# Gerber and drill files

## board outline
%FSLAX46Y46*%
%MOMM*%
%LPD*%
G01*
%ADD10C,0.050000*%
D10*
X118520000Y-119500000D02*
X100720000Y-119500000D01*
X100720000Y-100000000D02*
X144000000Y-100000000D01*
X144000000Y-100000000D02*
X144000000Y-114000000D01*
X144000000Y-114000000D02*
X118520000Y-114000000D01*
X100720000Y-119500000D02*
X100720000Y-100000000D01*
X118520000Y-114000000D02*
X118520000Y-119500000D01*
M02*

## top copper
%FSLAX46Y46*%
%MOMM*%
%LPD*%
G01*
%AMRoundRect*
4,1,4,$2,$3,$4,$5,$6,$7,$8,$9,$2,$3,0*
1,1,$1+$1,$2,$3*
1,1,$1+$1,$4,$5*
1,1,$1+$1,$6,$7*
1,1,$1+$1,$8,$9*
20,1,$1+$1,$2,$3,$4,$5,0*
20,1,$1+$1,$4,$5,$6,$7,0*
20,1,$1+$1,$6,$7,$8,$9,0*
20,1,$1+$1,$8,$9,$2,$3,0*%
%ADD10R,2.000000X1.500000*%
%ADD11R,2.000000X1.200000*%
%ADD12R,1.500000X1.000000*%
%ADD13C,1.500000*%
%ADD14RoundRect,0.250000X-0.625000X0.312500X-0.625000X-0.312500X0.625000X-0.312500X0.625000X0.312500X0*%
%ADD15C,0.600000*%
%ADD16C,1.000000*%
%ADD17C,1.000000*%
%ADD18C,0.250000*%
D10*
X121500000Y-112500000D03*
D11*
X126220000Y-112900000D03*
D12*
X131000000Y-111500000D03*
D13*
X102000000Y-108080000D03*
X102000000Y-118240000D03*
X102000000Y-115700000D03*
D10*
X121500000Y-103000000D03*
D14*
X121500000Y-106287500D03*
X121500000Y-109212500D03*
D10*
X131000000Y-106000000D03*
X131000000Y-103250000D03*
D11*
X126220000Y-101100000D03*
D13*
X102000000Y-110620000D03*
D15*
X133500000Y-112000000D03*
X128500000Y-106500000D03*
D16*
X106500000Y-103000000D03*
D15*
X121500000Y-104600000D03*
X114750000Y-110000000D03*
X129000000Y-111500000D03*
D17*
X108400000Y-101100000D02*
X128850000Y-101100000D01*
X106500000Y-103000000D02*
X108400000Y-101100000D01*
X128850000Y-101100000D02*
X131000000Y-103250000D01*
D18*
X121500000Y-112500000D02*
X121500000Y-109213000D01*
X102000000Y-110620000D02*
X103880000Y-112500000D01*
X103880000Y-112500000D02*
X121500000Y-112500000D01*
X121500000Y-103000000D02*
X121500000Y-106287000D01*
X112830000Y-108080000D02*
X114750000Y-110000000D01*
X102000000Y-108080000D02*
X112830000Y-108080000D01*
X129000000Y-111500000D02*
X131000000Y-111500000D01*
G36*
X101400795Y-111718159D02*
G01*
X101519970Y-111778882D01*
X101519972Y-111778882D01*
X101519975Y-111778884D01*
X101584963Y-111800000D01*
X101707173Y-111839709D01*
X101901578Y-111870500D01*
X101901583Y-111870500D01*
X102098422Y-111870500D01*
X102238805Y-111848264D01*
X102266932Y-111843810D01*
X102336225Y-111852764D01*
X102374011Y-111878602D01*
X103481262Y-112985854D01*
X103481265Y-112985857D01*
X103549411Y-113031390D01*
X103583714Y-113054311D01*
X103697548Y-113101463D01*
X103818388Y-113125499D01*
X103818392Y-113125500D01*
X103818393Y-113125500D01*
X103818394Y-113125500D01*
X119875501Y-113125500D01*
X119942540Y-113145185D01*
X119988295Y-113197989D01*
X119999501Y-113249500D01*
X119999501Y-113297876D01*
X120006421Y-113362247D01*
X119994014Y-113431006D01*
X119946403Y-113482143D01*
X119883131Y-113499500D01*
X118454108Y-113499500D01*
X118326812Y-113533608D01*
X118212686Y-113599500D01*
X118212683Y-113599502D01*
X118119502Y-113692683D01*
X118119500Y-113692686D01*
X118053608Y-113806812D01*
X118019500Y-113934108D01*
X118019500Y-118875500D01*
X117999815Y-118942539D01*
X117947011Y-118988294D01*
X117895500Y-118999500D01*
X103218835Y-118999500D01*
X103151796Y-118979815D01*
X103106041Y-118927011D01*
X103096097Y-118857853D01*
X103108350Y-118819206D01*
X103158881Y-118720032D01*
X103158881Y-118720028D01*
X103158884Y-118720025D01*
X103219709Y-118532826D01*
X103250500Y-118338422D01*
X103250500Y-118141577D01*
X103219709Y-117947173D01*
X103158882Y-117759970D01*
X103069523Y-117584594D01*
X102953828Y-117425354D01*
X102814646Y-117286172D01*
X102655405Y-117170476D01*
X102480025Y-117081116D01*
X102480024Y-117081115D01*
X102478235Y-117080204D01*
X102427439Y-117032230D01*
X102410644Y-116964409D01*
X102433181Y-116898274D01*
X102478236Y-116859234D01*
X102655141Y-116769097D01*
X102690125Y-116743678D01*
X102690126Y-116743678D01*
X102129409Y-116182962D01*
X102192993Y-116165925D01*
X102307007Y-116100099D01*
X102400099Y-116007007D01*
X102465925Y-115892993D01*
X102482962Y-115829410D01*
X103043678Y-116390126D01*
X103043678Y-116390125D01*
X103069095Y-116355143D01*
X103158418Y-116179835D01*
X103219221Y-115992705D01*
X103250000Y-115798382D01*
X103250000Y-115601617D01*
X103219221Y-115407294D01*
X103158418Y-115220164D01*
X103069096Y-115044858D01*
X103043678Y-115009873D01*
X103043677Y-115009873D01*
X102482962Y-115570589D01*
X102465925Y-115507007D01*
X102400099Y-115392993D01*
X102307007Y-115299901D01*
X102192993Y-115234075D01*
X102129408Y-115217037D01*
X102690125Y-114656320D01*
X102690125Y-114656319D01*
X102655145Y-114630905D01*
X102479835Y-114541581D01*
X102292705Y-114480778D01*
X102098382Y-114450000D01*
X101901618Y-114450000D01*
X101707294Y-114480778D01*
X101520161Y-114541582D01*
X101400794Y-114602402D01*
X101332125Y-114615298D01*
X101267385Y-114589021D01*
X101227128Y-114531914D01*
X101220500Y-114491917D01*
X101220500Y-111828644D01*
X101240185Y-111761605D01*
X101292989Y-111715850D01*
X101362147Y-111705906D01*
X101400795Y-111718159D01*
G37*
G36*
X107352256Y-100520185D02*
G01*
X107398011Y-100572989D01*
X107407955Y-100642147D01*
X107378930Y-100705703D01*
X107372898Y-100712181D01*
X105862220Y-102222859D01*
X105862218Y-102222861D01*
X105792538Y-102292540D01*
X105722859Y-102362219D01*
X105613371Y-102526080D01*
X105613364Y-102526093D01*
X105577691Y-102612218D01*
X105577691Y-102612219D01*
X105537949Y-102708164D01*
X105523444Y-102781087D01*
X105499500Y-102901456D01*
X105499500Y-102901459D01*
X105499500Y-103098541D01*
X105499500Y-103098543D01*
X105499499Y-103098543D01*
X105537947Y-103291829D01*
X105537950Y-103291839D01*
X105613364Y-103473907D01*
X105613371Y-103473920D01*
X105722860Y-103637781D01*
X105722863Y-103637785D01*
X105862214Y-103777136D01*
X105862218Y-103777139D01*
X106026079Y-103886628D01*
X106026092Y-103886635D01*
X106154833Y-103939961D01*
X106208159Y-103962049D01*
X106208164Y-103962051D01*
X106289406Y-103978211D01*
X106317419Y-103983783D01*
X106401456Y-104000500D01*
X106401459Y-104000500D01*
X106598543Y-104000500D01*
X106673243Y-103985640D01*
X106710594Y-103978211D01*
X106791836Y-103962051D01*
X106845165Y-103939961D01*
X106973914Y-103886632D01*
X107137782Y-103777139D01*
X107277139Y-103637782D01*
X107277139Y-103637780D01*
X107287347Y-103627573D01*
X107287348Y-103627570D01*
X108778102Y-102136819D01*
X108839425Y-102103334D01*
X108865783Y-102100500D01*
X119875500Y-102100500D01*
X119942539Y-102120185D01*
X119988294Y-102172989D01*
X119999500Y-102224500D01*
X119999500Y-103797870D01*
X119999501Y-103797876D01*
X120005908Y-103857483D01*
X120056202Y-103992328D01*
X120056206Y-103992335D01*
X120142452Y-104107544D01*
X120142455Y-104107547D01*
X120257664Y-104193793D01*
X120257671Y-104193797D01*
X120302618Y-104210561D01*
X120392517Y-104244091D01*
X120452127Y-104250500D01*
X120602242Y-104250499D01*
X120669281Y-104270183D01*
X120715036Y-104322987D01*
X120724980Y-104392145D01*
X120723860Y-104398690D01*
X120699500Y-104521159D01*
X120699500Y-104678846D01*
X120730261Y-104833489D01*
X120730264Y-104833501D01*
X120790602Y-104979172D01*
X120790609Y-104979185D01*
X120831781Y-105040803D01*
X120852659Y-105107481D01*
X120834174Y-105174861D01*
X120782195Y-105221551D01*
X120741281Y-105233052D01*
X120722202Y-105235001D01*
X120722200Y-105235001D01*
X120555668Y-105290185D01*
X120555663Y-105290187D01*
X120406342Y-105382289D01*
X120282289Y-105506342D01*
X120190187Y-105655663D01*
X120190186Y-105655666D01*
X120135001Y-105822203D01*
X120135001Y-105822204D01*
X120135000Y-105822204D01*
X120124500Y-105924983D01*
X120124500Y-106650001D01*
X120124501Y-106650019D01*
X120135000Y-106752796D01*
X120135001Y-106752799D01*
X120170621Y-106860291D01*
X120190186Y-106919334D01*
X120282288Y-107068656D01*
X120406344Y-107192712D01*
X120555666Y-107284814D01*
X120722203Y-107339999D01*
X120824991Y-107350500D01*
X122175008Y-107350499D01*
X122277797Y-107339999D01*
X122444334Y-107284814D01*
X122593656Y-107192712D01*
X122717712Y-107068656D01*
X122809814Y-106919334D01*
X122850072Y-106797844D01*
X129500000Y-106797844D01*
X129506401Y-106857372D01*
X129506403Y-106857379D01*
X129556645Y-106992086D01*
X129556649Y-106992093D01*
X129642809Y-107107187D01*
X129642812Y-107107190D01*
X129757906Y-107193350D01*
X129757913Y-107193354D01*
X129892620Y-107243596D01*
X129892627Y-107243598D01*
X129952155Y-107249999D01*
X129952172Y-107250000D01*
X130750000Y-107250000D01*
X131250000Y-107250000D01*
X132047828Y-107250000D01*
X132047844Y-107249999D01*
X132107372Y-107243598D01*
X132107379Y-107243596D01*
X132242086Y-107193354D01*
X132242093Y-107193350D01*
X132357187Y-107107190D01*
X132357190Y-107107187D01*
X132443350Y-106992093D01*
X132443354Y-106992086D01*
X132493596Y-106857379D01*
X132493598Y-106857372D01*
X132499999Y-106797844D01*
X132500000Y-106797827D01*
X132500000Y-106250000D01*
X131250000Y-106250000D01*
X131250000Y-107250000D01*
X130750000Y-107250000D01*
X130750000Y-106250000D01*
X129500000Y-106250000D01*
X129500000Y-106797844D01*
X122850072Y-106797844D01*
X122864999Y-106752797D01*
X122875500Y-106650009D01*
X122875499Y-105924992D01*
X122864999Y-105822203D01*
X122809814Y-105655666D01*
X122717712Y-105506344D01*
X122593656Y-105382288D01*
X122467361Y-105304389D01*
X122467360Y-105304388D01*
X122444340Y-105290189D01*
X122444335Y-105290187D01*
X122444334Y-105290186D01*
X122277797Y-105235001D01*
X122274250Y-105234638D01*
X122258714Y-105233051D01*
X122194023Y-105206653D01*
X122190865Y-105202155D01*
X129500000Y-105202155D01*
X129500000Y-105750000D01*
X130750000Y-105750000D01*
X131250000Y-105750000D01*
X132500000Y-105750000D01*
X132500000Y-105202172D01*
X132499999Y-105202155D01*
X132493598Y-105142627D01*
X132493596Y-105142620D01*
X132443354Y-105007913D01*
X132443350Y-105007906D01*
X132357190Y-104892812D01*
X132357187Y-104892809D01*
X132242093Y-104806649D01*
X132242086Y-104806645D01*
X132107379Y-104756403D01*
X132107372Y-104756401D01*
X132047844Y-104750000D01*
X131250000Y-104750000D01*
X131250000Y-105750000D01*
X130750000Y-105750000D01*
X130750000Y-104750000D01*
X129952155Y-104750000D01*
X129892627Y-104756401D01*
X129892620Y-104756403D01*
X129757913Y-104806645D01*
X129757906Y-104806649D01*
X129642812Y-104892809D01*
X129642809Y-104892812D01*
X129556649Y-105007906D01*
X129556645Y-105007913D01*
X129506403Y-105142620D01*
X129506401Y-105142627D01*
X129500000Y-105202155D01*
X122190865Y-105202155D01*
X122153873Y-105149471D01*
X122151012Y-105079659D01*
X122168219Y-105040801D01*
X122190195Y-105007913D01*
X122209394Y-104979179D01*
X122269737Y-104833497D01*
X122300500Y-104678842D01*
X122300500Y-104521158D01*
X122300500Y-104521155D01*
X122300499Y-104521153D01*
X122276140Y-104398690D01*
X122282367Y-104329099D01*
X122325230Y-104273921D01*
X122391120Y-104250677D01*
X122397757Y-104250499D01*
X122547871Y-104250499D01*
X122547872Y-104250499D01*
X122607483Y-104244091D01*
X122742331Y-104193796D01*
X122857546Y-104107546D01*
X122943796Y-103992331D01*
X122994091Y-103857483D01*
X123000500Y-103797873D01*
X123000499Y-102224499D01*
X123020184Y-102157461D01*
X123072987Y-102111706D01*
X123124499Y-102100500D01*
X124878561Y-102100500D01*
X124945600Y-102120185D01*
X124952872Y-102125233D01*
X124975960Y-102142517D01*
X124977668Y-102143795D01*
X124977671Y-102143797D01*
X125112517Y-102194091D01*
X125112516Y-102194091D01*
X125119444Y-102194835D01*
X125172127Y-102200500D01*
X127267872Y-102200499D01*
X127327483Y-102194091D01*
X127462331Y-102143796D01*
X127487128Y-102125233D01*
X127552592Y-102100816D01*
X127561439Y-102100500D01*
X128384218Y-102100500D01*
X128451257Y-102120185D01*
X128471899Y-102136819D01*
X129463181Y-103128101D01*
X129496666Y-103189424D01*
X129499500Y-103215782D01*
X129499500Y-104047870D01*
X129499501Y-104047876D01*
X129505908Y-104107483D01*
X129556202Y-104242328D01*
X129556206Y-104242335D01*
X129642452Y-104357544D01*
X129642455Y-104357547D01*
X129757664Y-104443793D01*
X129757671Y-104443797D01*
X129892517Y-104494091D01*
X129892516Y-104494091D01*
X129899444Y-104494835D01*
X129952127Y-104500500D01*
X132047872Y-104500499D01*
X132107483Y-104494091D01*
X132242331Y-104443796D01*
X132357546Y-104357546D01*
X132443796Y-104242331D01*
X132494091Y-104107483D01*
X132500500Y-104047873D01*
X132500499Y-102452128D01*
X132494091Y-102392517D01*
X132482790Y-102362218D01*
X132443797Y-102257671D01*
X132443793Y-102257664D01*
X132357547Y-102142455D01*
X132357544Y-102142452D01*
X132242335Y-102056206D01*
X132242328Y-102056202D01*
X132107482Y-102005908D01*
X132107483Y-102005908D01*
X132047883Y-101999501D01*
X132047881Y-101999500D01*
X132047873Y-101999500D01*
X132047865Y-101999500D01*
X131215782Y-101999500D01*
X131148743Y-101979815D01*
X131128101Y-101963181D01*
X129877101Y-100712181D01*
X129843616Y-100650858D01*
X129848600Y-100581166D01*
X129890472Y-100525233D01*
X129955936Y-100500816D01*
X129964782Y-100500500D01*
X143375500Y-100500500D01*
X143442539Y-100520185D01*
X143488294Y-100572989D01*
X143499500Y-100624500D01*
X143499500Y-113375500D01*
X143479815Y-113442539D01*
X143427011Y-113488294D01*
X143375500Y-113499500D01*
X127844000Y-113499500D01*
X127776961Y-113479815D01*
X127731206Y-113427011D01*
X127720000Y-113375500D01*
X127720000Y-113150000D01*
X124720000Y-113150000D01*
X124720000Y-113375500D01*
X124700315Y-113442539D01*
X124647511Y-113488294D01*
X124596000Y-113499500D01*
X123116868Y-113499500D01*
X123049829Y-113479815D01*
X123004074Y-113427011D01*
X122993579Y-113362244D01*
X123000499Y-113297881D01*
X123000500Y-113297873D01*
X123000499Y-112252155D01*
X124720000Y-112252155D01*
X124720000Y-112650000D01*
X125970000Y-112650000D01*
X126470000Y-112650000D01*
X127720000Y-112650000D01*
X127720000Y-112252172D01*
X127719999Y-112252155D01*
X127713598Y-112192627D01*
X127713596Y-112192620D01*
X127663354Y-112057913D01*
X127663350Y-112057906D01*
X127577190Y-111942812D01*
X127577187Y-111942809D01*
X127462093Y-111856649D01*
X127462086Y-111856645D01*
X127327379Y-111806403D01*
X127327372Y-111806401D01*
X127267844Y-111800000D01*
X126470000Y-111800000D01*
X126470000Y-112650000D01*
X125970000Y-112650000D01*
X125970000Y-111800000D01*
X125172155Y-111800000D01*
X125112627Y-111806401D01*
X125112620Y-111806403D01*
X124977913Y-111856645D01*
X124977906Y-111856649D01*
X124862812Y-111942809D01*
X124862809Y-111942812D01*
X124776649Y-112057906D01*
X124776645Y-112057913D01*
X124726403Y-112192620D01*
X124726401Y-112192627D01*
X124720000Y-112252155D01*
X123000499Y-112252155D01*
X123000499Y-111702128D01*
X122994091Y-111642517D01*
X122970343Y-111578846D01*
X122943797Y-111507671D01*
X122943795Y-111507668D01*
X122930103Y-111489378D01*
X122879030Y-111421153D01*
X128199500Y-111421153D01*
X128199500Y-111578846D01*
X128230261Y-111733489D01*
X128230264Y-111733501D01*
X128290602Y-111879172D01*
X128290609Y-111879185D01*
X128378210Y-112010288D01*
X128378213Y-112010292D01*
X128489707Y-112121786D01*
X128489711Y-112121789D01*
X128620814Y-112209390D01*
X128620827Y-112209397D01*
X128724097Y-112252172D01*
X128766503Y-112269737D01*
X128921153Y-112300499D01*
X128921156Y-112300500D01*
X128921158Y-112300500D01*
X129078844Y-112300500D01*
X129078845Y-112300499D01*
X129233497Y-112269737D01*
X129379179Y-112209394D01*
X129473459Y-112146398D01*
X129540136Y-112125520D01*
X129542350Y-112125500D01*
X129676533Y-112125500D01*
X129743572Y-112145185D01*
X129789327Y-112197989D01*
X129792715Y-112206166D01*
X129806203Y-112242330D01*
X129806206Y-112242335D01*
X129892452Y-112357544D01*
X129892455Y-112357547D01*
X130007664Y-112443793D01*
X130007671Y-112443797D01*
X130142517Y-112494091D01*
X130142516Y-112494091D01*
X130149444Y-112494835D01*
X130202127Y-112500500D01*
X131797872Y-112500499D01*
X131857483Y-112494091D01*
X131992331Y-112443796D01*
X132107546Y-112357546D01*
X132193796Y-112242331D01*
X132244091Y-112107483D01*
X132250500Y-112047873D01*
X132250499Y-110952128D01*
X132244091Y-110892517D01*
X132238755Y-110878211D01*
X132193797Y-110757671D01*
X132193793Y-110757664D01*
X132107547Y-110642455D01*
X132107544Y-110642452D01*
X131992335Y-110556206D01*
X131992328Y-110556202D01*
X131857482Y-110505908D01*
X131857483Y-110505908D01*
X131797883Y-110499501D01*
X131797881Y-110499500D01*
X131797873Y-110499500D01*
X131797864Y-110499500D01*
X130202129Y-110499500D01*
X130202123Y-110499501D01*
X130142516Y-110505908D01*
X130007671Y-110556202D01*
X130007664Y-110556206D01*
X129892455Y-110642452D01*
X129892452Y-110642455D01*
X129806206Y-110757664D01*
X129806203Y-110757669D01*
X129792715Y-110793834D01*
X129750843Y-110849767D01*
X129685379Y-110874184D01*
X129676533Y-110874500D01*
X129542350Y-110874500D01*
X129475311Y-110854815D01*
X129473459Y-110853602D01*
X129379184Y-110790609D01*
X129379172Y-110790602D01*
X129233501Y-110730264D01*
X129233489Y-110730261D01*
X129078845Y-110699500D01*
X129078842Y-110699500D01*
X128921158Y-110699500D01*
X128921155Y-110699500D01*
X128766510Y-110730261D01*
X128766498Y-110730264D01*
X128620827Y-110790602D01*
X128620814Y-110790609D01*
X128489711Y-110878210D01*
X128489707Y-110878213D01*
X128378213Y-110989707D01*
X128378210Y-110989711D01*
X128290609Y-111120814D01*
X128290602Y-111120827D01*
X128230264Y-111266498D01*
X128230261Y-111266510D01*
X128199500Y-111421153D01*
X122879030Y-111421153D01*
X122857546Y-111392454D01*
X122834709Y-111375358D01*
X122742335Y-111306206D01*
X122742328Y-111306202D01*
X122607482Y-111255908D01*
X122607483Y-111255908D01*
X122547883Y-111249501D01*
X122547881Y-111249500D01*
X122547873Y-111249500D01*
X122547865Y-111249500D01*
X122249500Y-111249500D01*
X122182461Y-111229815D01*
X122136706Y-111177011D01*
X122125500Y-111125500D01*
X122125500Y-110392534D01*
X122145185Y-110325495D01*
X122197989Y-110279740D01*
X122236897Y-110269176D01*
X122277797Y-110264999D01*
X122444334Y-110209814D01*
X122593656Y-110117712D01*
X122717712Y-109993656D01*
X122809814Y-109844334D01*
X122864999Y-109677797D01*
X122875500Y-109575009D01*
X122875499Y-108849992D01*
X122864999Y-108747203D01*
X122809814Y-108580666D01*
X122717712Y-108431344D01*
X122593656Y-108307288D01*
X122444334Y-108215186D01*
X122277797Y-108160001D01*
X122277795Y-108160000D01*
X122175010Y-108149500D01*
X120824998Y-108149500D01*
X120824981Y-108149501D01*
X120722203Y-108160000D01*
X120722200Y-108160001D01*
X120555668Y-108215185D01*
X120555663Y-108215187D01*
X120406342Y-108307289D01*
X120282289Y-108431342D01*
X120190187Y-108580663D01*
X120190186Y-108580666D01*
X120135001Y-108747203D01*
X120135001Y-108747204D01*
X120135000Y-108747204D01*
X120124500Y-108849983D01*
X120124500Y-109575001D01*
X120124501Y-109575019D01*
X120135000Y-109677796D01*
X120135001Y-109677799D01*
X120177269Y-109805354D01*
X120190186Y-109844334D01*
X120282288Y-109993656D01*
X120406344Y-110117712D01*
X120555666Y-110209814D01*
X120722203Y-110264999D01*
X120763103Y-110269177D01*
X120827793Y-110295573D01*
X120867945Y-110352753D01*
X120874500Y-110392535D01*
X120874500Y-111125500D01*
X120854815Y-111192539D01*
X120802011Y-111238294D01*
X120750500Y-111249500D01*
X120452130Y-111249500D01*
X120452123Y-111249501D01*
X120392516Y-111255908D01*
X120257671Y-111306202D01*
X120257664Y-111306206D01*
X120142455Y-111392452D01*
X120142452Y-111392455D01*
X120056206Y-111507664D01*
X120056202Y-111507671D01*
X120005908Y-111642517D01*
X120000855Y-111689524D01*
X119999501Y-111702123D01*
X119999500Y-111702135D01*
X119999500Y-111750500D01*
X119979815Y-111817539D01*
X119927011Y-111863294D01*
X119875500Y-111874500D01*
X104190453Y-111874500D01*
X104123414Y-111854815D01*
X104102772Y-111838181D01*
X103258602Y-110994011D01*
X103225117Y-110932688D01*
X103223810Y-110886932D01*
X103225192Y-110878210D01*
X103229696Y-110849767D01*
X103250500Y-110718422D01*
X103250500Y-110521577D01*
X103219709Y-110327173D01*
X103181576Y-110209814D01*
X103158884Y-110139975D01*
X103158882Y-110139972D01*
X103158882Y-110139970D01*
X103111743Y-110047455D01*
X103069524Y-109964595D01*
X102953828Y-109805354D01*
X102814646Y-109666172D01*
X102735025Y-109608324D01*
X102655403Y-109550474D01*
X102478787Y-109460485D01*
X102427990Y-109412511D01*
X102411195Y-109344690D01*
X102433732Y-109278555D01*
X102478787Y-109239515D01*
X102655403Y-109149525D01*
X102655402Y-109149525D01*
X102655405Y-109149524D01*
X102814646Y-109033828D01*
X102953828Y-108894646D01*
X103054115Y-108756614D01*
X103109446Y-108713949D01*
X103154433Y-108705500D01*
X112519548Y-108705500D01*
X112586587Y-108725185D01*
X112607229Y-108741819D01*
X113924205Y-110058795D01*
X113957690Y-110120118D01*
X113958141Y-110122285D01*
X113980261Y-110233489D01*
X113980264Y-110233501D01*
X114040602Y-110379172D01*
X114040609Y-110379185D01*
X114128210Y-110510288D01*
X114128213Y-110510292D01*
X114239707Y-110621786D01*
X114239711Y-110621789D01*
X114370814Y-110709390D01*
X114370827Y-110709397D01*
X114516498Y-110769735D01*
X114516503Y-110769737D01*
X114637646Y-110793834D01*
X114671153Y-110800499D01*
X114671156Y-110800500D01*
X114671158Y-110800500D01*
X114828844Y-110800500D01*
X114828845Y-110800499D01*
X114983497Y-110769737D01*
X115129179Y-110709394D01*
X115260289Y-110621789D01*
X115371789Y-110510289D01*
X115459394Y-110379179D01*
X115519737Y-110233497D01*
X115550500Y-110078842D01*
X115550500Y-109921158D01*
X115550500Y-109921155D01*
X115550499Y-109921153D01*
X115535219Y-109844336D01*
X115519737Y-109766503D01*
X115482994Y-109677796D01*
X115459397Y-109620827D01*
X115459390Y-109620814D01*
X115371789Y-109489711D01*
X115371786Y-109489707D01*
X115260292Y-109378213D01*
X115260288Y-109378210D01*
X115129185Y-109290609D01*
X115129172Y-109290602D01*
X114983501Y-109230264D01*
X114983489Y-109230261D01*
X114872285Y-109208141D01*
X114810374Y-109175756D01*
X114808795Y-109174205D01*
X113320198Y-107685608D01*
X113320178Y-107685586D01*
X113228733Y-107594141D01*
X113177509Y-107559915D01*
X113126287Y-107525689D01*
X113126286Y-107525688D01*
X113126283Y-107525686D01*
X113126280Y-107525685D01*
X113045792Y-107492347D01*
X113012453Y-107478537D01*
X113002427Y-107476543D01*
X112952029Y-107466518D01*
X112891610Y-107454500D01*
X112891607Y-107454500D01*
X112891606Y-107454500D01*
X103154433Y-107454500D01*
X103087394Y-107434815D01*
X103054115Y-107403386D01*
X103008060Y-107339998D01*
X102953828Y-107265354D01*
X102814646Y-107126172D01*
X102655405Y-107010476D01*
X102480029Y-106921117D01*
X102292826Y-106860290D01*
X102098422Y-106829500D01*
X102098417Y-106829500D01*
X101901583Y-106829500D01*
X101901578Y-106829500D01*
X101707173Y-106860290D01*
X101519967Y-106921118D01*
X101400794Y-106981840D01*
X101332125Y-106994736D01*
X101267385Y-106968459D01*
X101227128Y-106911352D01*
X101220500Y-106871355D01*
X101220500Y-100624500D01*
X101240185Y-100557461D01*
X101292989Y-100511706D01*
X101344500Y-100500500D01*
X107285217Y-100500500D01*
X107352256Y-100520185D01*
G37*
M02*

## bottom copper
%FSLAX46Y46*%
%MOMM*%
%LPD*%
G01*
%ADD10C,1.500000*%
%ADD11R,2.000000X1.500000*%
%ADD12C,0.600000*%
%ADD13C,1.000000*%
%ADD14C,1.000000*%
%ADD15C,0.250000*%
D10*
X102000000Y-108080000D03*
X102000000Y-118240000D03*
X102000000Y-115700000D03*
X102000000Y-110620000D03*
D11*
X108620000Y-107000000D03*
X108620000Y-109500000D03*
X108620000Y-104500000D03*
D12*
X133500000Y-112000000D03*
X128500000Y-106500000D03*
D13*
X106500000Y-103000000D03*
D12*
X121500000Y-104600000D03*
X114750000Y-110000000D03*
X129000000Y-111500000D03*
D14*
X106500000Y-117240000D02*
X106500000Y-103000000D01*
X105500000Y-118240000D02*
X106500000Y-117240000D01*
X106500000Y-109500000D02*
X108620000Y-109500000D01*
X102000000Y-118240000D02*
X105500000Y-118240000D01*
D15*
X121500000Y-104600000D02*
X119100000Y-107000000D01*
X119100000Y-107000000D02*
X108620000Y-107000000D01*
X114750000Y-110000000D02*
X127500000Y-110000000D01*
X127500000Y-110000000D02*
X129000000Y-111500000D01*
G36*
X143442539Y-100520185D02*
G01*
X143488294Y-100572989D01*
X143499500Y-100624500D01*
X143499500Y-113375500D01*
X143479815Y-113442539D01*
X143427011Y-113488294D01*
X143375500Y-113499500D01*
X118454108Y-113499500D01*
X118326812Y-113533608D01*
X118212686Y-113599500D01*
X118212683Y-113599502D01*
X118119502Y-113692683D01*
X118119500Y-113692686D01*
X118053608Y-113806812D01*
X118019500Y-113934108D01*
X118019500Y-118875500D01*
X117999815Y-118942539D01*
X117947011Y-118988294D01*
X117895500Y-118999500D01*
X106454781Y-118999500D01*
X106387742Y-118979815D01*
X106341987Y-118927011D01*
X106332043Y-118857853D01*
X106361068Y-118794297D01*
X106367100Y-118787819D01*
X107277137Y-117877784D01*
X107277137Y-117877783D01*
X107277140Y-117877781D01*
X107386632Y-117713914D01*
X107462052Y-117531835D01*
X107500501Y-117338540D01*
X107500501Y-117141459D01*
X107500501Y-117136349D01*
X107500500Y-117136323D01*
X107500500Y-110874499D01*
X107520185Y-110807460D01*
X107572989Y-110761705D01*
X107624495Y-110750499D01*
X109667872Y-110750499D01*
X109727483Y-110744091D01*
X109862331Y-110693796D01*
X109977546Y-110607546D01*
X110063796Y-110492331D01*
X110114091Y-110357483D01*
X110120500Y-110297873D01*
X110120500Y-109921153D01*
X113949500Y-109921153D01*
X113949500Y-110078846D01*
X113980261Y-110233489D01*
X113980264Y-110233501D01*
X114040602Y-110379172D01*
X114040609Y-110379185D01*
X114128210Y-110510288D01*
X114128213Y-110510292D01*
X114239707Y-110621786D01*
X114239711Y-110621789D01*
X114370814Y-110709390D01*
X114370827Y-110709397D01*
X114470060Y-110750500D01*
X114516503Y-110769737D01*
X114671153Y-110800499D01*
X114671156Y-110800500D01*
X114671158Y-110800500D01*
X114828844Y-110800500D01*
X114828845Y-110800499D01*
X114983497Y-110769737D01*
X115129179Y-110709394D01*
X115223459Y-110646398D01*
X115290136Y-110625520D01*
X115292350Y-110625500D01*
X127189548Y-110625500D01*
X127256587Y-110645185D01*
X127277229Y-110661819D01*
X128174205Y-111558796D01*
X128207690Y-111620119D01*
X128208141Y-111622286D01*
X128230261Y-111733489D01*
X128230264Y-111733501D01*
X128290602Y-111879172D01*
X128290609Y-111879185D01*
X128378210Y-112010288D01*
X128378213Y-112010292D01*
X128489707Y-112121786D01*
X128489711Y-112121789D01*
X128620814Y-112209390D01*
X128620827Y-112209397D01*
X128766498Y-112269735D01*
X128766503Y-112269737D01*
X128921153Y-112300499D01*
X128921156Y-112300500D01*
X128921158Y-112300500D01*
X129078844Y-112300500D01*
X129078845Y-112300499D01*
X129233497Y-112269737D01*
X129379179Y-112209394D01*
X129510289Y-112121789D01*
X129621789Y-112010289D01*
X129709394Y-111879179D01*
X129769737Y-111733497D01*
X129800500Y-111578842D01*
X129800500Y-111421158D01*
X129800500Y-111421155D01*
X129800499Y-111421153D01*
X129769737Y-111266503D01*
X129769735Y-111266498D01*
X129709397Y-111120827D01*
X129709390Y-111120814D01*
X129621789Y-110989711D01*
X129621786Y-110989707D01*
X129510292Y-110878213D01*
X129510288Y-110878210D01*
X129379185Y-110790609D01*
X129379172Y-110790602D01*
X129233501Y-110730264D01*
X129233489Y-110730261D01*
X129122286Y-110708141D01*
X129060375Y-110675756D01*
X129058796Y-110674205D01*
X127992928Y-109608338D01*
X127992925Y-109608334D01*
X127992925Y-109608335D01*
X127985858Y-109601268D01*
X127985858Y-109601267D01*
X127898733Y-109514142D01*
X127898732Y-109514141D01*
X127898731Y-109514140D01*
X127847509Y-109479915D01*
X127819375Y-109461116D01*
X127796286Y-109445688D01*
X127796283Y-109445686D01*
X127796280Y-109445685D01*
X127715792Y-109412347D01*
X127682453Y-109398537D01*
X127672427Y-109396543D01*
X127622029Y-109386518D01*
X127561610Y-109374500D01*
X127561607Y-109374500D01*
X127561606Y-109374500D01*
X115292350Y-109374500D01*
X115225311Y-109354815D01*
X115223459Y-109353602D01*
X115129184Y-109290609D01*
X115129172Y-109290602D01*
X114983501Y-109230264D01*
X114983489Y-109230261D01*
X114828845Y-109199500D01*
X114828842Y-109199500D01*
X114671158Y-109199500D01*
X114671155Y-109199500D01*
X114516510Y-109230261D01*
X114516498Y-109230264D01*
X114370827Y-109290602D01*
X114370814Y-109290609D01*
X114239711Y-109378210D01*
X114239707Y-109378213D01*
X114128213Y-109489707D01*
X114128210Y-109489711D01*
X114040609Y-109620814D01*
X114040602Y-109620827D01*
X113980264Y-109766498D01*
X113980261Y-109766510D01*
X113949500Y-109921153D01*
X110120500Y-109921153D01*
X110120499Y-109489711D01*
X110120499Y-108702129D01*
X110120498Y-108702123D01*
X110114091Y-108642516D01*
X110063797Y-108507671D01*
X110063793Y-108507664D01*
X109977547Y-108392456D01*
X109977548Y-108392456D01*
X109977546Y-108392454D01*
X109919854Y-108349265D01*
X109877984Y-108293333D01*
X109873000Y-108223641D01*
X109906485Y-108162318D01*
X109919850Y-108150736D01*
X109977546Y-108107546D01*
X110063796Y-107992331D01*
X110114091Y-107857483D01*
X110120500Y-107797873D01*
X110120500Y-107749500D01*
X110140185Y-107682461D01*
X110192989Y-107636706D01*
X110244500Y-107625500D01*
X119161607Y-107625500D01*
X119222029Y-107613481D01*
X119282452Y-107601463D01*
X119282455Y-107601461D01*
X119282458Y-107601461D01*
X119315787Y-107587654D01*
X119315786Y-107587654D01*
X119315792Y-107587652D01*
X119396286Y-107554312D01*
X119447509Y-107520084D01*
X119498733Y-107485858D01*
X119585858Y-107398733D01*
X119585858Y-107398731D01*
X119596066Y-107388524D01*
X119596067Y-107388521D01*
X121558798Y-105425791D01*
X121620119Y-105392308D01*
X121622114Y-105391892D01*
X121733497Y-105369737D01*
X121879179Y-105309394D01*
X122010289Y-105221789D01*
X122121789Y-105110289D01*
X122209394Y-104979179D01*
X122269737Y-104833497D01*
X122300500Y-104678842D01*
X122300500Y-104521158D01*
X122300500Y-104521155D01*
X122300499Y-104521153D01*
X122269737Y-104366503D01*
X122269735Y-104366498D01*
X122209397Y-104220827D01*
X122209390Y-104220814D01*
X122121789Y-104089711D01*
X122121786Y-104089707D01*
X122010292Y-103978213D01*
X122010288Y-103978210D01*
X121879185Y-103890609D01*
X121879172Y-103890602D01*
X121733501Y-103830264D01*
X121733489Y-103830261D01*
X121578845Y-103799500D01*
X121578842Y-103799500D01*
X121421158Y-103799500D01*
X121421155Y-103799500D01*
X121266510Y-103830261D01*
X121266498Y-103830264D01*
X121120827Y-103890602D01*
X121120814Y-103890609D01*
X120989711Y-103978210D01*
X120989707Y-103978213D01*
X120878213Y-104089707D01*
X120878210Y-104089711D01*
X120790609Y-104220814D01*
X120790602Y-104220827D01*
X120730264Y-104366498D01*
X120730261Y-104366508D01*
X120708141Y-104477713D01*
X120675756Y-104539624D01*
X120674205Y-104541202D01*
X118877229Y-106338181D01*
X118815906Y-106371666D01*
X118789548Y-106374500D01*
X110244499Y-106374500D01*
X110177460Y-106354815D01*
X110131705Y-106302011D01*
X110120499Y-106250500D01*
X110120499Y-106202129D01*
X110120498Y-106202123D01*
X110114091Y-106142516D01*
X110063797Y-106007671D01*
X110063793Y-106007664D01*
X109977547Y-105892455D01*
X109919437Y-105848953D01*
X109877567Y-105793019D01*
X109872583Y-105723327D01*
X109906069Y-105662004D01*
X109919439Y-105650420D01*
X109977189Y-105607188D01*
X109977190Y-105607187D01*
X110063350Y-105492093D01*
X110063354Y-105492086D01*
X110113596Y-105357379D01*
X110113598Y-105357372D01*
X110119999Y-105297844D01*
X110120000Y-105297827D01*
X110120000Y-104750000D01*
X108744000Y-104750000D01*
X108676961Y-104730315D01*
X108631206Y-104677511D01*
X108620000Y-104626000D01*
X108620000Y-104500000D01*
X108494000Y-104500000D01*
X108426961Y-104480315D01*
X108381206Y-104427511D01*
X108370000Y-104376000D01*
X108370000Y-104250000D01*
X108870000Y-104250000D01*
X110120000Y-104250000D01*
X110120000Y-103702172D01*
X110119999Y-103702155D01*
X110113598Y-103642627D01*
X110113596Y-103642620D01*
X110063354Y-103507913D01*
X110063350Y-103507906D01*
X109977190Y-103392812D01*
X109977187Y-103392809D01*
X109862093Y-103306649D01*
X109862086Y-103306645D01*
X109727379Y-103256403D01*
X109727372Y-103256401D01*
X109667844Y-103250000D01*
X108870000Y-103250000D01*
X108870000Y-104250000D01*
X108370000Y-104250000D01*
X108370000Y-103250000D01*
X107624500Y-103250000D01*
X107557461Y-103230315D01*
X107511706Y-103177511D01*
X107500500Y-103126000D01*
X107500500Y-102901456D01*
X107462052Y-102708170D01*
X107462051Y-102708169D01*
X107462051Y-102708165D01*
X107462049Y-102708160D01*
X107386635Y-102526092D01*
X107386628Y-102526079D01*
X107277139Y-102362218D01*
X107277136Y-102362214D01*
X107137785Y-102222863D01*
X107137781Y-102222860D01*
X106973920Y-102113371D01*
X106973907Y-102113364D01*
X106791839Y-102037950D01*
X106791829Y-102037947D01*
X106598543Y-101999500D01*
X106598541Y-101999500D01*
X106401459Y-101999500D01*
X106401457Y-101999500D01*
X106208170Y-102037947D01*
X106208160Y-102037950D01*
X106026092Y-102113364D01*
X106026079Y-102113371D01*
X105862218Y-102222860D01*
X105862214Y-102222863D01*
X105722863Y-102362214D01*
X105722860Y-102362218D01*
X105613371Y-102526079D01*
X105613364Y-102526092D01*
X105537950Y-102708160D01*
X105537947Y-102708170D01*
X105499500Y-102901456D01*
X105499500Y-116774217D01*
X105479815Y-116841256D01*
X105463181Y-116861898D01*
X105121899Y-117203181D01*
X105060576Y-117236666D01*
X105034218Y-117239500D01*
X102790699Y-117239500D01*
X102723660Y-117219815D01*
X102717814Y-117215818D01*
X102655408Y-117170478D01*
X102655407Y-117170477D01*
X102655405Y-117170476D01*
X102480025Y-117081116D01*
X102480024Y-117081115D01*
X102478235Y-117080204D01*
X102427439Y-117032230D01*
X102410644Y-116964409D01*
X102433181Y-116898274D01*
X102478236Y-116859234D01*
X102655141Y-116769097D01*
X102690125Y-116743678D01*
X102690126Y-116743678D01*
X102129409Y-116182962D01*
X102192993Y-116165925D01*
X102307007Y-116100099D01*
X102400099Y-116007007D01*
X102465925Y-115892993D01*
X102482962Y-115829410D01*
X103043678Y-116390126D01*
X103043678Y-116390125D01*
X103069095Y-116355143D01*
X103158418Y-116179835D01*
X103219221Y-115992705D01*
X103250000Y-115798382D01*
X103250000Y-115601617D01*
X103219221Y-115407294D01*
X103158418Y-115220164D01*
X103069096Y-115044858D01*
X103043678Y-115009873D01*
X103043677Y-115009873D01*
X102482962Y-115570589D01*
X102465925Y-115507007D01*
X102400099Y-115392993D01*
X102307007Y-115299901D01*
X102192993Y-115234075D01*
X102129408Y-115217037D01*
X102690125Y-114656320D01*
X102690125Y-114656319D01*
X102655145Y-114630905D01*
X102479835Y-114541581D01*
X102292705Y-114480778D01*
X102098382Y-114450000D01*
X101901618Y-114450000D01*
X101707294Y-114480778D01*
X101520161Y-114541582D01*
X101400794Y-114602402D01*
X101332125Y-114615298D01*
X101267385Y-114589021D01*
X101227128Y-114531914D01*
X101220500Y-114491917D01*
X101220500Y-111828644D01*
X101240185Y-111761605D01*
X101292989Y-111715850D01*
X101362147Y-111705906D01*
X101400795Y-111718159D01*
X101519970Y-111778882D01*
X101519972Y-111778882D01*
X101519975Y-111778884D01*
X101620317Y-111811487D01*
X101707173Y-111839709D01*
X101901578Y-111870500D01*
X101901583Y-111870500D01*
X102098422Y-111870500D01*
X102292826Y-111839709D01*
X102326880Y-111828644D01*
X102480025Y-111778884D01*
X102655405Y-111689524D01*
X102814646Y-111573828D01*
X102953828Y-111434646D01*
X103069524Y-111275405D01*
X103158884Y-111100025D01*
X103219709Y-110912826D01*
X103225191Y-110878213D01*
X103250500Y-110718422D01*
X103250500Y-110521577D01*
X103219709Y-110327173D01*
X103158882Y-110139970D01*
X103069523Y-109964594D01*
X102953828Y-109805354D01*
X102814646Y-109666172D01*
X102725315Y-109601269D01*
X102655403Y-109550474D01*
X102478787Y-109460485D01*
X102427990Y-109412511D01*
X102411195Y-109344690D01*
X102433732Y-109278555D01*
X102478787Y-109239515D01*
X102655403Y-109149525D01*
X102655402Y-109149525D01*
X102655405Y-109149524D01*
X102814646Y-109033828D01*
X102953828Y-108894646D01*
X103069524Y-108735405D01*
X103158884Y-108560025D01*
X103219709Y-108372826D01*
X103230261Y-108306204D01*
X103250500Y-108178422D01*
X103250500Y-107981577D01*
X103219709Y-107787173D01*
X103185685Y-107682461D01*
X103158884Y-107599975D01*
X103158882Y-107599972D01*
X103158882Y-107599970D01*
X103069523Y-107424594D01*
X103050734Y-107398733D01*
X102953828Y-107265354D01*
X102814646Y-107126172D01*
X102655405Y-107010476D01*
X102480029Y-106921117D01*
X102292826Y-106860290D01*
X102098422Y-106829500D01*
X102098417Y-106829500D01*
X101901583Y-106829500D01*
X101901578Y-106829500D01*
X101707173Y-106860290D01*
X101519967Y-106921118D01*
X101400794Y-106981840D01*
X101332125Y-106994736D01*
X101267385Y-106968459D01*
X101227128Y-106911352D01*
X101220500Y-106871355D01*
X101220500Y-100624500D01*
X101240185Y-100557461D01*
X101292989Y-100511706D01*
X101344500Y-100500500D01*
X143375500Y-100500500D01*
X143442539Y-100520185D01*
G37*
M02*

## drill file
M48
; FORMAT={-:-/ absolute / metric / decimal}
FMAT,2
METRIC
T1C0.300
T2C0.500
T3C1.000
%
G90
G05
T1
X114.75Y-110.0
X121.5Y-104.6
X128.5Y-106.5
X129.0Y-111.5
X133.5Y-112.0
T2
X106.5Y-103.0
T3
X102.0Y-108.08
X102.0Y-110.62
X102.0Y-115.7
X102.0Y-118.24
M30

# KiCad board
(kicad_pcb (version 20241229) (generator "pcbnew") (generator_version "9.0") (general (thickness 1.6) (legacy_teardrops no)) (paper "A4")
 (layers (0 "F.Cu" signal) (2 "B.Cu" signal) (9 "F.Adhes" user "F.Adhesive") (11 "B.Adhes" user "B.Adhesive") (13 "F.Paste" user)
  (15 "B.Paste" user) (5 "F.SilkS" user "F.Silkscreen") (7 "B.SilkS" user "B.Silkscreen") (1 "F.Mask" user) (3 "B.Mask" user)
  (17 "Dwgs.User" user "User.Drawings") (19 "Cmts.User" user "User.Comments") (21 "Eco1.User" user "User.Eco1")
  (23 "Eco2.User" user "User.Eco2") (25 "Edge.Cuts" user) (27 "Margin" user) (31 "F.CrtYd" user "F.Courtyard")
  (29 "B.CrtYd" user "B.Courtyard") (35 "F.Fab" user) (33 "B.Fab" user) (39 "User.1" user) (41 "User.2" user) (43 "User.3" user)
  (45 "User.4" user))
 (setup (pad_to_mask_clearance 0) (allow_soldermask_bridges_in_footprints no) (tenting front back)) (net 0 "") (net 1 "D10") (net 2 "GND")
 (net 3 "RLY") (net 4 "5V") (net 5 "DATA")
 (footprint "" (layer "F.Cu") (at 121.5 112.5)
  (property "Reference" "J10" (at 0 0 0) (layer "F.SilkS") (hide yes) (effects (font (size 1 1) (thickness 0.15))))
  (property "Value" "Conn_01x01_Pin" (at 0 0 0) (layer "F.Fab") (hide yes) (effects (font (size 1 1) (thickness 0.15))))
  (pad "1" smd rect (at 0 0) (size 2 1.5) (layers "F.Cu" "F.Mask") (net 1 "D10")))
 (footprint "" (layer "F.Cu") (at 126.22 112.9)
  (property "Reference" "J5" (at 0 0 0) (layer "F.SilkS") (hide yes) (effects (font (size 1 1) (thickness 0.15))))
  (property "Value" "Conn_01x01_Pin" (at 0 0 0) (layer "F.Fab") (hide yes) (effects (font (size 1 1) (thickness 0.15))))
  (pad "1" smd rect (at 0 0) (size 2 1.2) (layers "F.Cu" "F.Mask") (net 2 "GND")))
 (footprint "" (layer "F.Cu") (at 131 111.5)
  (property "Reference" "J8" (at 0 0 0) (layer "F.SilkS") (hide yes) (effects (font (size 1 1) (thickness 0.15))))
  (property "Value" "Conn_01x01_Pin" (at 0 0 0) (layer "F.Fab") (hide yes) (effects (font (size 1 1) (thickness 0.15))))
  (pad "1" smd rect (at 0 0) (size 1.5 1) (layers "F.Cu" "F.Mask") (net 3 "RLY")))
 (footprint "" (layer "F.Cu") (at 102 108.08)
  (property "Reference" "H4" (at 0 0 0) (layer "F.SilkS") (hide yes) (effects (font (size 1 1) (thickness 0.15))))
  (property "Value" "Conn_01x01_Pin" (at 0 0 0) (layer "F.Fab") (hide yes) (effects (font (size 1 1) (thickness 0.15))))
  (pad "1" thru_hole circle (at 0 0) (size 1.5 1.5) (drill 1) (layers "*.Cu" "*.Mask") (remove_unused_layers no) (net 3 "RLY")))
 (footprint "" (layer "F.Cu") (at 102 118.24)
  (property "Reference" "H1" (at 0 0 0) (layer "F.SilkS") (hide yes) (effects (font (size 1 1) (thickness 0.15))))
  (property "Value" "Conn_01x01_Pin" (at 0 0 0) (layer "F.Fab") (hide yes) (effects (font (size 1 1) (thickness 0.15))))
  (pad "1" thru_hole circle (at 0 0) (size 1.5 1.5) (drill 1) (layers "*.Cu" "*.Mask") (remove_unused_layers no) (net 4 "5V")))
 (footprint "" (layer "F.Cu") (at 102 115.7)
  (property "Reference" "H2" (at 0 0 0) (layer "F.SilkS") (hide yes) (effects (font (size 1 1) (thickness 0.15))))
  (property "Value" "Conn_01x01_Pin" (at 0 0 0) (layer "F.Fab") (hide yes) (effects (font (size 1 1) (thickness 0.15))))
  (pad "1" thru_hole circle (at 0 0) (size 1.5 1.5) (drill 1) (layers "*.Cu" "*.Mask") (remove_unused_layers no) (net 2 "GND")))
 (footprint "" (layer "F.Cu") (at 121.5 103)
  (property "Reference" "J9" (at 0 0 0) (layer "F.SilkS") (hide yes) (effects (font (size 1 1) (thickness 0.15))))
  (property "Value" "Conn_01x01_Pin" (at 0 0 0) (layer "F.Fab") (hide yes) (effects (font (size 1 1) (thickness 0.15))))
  (pad "1" smd rect (at 0 0) (size 2 1.5) (layers "F.Cu" "F.Mask") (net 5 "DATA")))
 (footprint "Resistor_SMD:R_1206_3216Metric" (layer "F.Cu") (at 121.5 107.75 -90)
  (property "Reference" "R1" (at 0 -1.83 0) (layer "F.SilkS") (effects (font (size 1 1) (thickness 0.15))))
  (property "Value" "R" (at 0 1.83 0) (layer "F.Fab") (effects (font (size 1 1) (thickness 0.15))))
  (pad "1" smd roundrect (at -1.4625 0 270) (size 1.125 1.75) (layers "F.Cu" "F.Mask" "F.Paste") (roundrect_rratio 0.222222) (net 5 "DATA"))
  (pad "2" smd roundrect (at 1.4625 0 270) (size 1.125 1.75) (layers "F.Cu" "F.Mask" "F.Paste") (roundrect_rratio 0.222222) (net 1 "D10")))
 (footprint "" (layer "F.Cu") (at 131 106)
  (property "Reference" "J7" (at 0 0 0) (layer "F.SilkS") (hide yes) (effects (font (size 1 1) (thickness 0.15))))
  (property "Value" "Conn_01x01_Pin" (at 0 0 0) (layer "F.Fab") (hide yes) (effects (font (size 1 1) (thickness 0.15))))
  (pad "1" smd rect (at 0 0) (size 2 1.5) (layers "F.Cu" "F.Mask") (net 2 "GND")))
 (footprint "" (layer "F.Cu") (at 131 103.25)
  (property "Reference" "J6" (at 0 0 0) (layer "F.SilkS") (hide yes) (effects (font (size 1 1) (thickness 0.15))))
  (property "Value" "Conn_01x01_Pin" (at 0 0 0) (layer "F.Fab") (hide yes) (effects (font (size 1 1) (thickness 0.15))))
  (pad "1" smd rect (at 0 0) (size 2 1.5) (layers "F.Cu" "F.Mask") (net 4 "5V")))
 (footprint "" (layer "F.Cu") (at 126.22 101.1)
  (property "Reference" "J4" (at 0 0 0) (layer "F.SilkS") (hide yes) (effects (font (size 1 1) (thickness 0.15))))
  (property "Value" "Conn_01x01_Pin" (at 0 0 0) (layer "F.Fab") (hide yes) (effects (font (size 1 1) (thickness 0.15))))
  (pad "1" smd rect (at 0 0) (size 2 1.2) (layers "F.Cu" "F.Mask") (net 4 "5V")))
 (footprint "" (layer "F.Cu") (at 102 110.62)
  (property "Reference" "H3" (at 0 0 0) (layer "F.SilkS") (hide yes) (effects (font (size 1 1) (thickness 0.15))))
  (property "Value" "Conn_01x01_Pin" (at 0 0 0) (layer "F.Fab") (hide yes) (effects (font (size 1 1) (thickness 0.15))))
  (pad "1" thru_hole circle (at 0 0) (size 1.5 1.5) (drill 1) (layers "*.Cu" "*.Mask") (remove_unused_layers no) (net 1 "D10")))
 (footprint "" (layer "B.Cu") (at 108.62 107)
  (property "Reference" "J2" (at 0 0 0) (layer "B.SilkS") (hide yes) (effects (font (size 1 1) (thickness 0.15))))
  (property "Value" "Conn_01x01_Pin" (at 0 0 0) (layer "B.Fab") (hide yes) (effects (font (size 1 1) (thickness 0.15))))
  (pad "1" smd rect (at 0 0) (size 2 1.5) (layers "B.Cu" "B.Mask") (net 5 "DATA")))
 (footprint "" (layer "B.Cu") (at 108.62 109.5)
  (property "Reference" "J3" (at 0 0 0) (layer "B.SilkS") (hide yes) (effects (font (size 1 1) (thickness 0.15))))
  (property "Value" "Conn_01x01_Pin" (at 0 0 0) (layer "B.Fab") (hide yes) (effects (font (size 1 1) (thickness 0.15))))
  (pad "1" smd rect (at 0 0) (size 2 1.5) (layers "B.Cu" "B.Mask") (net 4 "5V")))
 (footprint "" (layer "B.Cu") (at 108.62 104.5)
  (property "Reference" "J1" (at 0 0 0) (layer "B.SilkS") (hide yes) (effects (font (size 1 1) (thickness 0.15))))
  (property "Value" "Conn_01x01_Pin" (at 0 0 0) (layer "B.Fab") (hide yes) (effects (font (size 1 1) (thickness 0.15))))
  (pad "1" smd rect (at 0 0) (size 2 1.5) (layers "B.Cu" "B.Mask") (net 2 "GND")))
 (gr_line (start 118.52 119.5) (end 100.72 119.5) (stroke (width 0.05) (type default)) (layer "Edge.Cuts"))
 (gr_line (start 100.72 100) (end 144 100) (stroke (width 0.05) (type default)) (layer "Edge.Cuts"))
 (gr_line (start 144 100) (end 144 114) (stroke (width 0.05) (type default)) (layer "Edge.Cuts"))
 (gr_line (start 144 114) (end 118.52 114) (stroke (width 0.05) (type default)) (layer "Edge.Cuts"))
 (gr_line (start 100.72 119.5) (end 100.72 100) (stroke (width 0.05) (type default)) (layer "Edge.Cuts"))
 (gr_line (start 118.52 114) (end 118.52 119.5) (stroke (width 0.05) (type default)) (layer "Edge.Cuts"))
 (via (at 133.5 112) (size 0.6) (drill 0.3) (layers "F.Cu" "B.Cu") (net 2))
 (via (at 128.5 106.5) (size 0.6) (drill 0.3) (layers "F.Cu" "B.Cu") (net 2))
 (segment (start 108.4 101.1) (end 128.85 101.1) (width 1) (layer "F.Cu") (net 4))
 (segment (start 106.5 103) (end 108.4 101.1) (width 1) (layer "F.Cu") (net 4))
 (segment (start 128.85 101.1) (end 131 103.25) (width 1) (layer "F.Cu") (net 4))
 (via (at 106.5 103) (size 1) (drill 0.5) (layers "F.Cu" "B.Cu") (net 4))
 (segment (start 106.5 117.24) (end 106.5 103) (width 1) (layer "B.Cu") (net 4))
 (segment (start 105.5 118.24) (end 106.5 117.24) (width 1) (layer "B.Cu") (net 4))
 (segment (start 106.5 109.5) (end 108.62 109.5) (width 1) (layer "B.Cu") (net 4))
 (segment (start 102 118.24) (end 105.5 118.24) (width 1) (layer "B.Cu") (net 4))
 (segment (start 121.5 112.5) (end 121.5 109.213) (width 0.25) (layer "F.Cu") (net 1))
 (segment (start 102 110.62) (end 103.88 112.5) (width 0.25) (layer "F.Cu") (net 1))
 (segment (start 103.88 112.5) (end 121.5 112.5) (width 0.25) (layer "F.Cu") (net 1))
 (segment (start 121.5 103) (end 121.5 106.287) (width 0.25) (layer "F.Cu") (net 5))
 (via (at 121.5 104.6) (size 0.6) (drill 0.3) (layers "F.Cu" "B.Cu") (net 5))
 (segment (start 121.5 104.6) (end 119.1 107) (width 0.25) (layer "B.Cu") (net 5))
 (segment (start 119.1 107) (end 108.62 107) (width 0.25) (layer "B.Cu") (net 5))
 (segment (start 112.83 108.08) (end 114.75 110) (width 0.25) (layer "F.Cu") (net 3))
 (segment (start 102 108.08) (end 112.83 108.08) (width 0.25) (layer "F.Cu") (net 3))
 (segment (start 129 111.5) (end 131 111.5) (width 0.25) (layer "F.Cu") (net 3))
 (via (at 114.75 110) (size 0.6) (drill 0.3) (layers "F.Cu" "B.Cu") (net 3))
 (via (at 129 111.5) (size 0.6) (drill 0.3) (layers "F.Cu" "B.Cu") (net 3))
 (segment (start 114.75 110) (end 127.5 110) (width 0.25) (layer "B.Cu") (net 3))
 (segment (start 127.5 110) (end 129 111.5) (width 0.25) (layer "B.Cu") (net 3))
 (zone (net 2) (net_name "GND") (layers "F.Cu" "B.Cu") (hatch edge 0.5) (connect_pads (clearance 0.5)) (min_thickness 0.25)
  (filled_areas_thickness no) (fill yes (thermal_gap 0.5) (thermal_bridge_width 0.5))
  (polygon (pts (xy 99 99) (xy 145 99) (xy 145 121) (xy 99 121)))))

